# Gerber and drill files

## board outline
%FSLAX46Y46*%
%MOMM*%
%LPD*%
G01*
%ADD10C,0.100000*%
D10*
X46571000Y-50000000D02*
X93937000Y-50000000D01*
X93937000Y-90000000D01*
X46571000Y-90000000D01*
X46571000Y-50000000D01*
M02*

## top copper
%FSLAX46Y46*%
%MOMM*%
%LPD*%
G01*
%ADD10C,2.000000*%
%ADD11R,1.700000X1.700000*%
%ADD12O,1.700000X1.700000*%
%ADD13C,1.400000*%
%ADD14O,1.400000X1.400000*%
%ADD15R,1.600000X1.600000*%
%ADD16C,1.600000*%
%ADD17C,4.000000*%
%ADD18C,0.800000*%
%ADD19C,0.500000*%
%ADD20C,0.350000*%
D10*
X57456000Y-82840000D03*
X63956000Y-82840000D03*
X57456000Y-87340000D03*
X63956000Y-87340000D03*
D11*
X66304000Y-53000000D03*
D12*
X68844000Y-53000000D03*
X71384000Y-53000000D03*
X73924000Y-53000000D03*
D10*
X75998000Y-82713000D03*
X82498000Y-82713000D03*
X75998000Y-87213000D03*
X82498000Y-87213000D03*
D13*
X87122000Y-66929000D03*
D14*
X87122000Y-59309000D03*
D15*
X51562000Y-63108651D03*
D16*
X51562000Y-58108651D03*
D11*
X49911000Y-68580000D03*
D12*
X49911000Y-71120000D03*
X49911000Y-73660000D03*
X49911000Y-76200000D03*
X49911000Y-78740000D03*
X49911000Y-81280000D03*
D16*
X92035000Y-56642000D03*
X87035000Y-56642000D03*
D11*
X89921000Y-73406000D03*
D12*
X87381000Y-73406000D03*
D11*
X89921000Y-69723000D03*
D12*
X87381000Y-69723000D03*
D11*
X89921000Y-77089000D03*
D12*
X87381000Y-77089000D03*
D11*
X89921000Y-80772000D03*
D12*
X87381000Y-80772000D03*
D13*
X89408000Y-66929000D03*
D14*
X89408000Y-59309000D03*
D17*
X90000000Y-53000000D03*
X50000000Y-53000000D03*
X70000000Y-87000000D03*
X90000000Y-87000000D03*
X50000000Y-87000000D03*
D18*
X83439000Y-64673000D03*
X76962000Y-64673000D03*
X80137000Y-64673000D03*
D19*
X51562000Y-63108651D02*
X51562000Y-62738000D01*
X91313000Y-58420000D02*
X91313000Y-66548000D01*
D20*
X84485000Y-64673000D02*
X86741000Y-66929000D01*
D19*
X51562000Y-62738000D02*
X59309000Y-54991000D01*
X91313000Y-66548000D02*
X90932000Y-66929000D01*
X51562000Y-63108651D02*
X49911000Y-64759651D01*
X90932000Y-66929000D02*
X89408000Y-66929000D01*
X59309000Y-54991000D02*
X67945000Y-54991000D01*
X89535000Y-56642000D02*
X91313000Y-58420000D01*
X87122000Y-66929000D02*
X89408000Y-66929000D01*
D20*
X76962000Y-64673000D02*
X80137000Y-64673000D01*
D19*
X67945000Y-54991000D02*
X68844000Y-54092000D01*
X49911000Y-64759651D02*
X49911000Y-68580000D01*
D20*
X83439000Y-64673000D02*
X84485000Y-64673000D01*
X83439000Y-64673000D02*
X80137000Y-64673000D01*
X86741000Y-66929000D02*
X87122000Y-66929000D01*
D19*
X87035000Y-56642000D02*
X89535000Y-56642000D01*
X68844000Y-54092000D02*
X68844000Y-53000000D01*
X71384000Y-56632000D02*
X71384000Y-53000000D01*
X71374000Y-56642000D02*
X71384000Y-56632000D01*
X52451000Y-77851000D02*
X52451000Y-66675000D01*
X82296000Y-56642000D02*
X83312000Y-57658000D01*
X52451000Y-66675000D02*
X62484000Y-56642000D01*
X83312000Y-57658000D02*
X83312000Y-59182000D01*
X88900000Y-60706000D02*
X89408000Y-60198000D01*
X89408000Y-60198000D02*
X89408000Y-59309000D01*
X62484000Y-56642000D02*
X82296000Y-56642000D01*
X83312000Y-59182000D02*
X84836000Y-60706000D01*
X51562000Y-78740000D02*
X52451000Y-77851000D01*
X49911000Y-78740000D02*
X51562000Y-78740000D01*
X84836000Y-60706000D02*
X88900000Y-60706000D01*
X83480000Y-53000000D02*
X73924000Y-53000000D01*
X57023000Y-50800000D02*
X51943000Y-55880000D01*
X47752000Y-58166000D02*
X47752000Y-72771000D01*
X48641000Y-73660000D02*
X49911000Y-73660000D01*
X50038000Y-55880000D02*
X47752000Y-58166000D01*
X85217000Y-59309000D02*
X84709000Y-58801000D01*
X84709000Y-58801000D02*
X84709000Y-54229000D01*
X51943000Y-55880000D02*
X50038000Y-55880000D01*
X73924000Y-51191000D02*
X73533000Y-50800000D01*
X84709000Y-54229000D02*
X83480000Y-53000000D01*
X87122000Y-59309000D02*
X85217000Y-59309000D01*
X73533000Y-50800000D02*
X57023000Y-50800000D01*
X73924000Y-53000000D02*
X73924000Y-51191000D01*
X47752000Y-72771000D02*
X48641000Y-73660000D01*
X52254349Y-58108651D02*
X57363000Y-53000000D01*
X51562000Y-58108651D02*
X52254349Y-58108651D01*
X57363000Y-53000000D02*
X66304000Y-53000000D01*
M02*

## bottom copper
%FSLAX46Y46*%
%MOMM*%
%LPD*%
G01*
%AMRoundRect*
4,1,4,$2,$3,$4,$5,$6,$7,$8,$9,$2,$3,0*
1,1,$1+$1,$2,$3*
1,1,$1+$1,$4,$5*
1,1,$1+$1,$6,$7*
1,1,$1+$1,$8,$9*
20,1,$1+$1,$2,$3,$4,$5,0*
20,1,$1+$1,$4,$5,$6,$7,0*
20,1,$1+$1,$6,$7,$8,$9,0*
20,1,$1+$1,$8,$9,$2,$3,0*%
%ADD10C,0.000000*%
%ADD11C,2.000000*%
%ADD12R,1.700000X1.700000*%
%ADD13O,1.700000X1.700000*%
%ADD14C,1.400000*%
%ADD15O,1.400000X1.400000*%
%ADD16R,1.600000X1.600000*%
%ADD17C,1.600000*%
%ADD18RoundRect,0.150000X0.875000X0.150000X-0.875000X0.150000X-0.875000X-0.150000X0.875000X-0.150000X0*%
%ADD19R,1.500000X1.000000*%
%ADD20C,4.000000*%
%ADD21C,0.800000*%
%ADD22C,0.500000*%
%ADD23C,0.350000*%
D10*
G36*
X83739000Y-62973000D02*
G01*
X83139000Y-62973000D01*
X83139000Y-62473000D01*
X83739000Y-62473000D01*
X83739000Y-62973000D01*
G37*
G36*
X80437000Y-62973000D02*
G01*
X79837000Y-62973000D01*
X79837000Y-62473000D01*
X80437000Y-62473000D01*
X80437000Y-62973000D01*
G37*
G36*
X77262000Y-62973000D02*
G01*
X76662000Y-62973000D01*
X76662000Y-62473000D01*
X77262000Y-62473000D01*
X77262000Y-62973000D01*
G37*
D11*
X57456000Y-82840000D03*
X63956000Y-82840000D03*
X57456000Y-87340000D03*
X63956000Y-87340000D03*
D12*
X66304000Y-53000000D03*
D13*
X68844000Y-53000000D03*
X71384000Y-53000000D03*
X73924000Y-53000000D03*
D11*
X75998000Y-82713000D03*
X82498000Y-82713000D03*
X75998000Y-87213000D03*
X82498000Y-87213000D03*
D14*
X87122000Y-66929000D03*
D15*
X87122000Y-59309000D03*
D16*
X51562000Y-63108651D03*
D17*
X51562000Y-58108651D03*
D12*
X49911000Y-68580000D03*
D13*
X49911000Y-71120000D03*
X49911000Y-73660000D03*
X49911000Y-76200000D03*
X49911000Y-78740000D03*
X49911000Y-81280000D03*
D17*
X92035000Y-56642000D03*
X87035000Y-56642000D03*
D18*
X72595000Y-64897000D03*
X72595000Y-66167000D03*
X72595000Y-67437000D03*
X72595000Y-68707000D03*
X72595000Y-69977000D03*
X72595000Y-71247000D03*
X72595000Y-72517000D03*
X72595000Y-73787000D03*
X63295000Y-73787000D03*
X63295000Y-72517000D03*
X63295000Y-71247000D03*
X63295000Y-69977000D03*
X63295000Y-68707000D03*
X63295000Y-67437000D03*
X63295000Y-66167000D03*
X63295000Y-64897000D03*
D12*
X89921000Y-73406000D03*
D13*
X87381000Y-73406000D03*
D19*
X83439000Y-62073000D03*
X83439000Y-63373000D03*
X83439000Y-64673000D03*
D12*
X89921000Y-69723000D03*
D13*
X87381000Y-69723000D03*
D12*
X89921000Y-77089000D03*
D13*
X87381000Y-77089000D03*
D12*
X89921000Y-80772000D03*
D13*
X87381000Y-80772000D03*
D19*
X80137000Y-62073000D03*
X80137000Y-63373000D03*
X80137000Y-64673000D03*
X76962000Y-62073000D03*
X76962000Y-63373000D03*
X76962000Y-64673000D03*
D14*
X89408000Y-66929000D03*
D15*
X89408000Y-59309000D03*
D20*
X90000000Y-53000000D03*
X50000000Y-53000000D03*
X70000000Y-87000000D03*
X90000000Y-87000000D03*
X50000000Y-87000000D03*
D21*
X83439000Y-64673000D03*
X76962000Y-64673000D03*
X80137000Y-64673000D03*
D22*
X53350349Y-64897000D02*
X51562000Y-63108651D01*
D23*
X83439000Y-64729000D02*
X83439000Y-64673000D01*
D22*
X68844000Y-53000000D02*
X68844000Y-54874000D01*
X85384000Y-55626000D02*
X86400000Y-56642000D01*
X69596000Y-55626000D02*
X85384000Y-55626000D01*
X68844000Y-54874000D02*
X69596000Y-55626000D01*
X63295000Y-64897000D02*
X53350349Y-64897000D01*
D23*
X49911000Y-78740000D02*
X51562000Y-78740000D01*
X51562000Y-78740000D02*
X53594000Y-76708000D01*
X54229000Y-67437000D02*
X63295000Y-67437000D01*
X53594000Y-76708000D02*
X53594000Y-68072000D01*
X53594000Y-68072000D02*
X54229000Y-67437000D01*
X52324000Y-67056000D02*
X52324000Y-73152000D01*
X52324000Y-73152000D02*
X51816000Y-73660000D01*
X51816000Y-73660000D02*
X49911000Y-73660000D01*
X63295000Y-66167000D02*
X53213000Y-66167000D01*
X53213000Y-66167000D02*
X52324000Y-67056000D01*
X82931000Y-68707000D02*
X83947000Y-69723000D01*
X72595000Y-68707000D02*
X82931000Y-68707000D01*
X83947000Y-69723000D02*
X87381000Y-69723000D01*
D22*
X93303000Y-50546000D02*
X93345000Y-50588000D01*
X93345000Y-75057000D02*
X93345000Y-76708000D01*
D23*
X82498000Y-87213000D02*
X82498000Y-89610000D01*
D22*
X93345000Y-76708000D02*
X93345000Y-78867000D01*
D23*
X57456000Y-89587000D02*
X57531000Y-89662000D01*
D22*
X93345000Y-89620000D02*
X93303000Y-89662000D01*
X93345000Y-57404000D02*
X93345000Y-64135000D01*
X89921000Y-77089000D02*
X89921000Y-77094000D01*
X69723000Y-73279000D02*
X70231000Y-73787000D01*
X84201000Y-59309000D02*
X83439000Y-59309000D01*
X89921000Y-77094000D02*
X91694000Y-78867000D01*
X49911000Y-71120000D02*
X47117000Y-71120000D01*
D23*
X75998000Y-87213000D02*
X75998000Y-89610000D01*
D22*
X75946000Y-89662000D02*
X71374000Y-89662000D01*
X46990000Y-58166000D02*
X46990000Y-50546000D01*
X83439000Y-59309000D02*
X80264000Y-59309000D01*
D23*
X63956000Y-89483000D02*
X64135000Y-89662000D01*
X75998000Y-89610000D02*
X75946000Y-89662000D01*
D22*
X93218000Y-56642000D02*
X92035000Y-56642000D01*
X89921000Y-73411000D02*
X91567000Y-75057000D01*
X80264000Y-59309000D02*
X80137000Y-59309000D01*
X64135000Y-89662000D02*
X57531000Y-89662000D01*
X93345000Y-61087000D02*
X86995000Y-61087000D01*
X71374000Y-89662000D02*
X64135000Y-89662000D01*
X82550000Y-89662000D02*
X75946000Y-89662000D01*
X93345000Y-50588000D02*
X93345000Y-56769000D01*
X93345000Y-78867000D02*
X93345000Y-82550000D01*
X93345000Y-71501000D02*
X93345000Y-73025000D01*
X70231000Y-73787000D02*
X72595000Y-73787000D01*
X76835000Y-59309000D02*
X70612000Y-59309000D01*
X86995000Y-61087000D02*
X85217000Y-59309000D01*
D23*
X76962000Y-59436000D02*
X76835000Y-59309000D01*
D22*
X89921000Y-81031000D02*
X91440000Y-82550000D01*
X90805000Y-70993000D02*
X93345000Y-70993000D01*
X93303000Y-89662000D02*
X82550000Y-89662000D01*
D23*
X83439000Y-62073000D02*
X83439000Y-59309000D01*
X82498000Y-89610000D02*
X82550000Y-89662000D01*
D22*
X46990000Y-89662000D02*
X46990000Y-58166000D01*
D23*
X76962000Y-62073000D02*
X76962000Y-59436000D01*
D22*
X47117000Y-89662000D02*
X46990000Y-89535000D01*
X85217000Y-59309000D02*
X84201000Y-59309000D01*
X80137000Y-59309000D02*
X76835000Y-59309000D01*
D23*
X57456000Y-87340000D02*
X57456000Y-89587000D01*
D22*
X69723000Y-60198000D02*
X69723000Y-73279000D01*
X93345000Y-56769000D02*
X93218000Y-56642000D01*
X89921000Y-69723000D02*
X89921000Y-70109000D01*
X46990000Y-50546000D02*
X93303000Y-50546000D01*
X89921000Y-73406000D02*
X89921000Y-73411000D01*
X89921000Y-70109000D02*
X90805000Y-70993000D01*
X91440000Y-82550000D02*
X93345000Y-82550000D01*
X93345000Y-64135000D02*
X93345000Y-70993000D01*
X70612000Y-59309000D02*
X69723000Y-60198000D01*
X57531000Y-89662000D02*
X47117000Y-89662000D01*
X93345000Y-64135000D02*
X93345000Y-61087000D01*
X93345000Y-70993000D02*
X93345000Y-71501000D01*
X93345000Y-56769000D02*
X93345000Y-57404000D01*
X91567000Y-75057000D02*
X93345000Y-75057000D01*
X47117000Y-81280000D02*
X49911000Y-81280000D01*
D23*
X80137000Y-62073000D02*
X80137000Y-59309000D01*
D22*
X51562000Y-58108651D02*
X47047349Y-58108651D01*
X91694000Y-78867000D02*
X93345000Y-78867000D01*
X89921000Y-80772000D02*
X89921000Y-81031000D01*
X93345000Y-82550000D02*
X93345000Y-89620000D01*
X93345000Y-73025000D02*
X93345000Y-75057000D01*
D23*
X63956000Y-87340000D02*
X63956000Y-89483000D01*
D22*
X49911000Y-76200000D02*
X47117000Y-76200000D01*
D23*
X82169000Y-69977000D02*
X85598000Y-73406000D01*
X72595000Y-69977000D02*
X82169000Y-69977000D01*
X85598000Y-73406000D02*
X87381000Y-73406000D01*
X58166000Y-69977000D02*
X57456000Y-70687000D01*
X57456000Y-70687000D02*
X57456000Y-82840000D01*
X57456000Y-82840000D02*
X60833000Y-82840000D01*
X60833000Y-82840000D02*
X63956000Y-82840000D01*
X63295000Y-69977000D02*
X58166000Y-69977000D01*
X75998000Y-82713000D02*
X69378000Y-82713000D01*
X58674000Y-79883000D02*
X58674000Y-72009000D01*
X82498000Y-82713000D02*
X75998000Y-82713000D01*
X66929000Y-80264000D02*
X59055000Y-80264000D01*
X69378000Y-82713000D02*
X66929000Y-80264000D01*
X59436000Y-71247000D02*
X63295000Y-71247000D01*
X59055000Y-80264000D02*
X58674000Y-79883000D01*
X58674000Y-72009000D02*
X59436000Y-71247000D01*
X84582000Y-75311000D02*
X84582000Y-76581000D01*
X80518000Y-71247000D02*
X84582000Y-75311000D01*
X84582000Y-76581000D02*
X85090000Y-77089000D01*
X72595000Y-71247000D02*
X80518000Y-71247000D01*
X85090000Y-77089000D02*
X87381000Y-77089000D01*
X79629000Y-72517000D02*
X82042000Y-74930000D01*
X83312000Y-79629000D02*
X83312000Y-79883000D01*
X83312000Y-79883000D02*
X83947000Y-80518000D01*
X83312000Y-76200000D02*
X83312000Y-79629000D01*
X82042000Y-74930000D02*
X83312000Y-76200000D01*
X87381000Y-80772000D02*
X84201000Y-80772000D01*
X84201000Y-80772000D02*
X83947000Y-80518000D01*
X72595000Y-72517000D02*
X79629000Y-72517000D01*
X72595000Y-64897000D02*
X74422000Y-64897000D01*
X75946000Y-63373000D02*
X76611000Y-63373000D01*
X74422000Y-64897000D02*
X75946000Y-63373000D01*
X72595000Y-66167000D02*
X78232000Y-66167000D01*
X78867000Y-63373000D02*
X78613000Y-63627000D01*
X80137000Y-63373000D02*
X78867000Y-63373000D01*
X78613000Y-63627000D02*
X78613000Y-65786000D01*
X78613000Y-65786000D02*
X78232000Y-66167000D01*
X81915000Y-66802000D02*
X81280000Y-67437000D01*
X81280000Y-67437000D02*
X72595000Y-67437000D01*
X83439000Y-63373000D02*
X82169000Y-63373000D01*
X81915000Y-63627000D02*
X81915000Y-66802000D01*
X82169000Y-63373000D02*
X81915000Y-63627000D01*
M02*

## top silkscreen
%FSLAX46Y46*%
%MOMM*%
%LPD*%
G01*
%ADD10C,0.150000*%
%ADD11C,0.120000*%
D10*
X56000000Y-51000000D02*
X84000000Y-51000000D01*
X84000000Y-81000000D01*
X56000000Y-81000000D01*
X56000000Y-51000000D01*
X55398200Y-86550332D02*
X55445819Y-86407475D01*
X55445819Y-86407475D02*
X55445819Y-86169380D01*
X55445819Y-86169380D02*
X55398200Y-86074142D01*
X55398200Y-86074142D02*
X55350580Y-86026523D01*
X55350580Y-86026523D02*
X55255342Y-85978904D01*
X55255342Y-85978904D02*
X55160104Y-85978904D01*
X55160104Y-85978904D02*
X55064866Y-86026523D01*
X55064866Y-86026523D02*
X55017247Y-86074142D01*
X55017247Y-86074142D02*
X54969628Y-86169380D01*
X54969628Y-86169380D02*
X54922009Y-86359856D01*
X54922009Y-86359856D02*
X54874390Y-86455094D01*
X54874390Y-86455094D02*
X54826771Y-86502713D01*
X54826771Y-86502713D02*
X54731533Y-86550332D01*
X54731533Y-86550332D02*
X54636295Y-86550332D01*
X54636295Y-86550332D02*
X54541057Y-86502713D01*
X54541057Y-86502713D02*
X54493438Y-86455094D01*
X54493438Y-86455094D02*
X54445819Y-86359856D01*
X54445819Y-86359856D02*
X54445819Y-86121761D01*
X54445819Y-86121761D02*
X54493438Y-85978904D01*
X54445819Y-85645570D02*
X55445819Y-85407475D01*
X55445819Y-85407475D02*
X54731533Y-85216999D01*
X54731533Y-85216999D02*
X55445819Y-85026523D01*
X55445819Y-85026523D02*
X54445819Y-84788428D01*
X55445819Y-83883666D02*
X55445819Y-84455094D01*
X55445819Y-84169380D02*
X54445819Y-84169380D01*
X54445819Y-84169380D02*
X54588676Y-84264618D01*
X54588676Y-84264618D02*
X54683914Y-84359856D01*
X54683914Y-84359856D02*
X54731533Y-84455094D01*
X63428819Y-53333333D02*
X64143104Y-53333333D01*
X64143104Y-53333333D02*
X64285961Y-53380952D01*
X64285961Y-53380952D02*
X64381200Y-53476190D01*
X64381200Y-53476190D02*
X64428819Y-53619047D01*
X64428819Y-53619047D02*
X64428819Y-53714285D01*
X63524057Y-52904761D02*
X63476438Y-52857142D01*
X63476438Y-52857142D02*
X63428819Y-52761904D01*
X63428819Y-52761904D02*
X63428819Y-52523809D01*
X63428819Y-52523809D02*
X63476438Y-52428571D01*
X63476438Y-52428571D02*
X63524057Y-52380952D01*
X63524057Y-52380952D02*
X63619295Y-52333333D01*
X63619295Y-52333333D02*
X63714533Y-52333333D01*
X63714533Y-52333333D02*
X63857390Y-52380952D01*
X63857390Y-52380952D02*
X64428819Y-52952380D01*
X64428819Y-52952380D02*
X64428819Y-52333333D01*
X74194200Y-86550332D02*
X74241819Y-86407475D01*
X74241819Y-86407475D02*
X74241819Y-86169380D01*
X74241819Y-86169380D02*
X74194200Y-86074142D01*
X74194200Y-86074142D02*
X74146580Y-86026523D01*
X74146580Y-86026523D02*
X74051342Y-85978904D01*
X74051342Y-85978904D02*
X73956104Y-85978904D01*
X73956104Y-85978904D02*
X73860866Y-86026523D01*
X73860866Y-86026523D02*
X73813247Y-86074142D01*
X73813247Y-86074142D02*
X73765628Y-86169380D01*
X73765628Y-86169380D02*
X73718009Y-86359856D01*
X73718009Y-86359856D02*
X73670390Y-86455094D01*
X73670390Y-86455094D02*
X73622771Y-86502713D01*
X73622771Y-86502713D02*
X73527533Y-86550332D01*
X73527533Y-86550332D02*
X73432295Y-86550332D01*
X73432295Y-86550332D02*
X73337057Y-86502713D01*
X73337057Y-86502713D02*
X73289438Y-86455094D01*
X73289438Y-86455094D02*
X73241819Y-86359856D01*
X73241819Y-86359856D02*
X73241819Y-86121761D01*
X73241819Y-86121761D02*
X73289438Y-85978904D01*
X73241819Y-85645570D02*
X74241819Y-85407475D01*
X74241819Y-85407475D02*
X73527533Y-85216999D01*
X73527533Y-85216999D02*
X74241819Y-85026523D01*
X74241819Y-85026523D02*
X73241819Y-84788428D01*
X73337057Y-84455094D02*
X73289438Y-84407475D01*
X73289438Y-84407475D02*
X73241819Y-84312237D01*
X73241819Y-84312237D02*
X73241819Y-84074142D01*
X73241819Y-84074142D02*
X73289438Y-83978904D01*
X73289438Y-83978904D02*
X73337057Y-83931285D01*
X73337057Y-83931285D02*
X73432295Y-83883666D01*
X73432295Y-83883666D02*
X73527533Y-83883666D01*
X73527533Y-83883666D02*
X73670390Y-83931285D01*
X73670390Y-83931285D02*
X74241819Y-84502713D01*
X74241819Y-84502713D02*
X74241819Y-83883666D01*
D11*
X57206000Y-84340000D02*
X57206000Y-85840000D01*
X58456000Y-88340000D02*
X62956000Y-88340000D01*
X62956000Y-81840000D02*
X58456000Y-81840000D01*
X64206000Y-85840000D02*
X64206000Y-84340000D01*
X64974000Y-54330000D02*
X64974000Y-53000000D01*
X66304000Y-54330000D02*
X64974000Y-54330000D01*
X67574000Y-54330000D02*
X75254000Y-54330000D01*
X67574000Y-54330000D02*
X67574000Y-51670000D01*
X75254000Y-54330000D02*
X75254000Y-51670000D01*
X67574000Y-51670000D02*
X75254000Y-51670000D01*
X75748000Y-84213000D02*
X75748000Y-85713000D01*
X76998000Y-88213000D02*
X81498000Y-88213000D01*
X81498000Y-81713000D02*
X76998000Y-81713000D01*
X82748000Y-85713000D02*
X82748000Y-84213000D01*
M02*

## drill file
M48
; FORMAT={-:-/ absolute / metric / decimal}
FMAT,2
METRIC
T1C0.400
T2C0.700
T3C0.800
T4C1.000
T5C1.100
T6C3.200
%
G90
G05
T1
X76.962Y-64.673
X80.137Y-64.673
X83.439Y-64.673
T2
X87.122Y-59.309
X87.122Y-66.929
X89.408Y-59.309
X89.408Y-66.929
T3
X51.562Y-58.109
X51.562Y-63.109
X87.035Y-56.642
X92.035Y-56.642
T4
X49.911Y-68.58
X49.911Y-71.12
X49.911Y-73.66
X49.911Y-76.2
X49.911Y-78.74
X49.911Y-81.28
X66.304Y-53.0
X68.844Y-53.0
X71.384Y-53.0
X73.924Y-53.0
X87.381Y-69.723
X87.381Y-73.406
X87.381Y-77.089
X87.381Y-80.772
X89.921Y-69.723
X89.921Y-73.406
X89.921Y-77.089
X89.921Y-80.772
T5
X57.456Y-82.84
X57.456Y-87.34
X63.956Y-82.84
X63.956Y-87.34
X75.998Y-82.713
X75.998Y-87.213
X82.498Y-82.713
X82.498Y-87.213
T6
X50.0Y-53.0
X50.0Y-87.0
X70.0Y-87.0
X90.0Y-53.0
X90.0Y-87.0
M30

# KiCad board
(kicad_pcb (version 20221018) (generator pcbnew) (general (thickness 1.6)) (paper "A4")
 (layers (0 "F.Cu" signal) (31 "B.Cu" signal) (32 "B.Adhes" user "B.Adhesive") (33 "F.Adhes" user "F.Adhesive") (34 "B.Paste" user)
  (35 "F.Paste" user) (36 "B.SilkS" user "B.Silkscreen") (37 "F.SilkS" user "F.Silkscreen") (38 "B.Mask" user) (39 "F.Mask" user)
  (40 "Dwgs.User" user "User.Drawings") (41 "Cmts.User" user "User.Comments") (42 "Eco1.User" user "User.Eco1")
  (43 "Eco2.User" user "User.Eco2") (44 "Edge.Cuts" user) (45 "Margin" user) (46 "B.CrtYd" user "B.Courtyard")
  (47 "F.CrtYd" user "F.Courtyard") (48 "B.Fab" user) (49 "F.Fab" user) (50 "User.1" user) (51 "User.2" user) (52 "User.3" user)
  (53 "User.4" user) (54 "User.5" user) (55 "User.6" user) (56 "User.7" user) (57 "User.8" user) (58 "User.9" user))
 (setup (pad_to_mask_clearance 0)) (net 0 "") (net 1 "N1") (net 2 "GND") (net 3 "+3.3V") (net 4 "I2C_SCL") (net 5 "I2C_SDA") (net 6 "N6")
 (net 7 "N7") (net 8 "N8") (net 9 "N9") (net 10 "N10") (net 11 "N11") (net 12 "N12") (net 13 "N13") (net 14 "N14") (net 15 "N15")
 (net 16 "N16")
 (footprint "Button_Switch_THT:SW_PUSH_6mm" (layer "F.Cu") (at 57.456 82.84)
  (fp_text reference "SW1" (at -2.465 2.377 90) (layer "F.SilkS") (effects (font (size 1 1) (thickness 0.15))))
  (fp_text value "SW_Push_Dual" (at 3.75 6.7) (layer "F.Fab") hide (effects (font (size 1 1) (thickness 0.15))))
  (fp_line (start -0.25 1.5) (end -0.25 3) (stroke (width 0.12) (type solid)) (layer "F.SilkS"))
  (fp_line (start 1 5.5) (end 5.5 5.5) (stroke (width 0.12) (type solid)) (layer "F.SilkS"))
  (fp_line (start 5.5 -1) (end 1 -1) (stroke (width 0.12) (type solid)) (layer "F.SilkS"))
  (fp_line (start 6.75 3) (end 6.75 1.5) (stroke (width 0.12) (type solid)) (layer "F.SilkS"))
  (pad "1" thru_hole circle (at 0 0 90) (size 2 2) (drill 1.1) (layers "*.Cu" "*.Mask") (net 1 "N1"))
  (pad "1" thru_hole circle (at 6.5 0 90) (size 2 2) (drill 1.1) (layers "*.Cu" "*.Mask") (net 1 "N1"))
  (pad "2" thru_hole circle (at 0 4.5 90) (size 2 2) (drill 1.1) (layers "*.Cu" "*.Mask") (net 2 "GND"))
  (pad "2" thru_hole circle (at 6.5 4.5 90) (size 2 2) (drill 1.1) (layers "*.Cu" "*.Mask") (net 2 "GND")))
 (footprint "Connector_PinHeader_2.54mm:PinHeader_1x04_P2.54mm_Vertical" (layer "F.Cu") (at 66.304 53 90)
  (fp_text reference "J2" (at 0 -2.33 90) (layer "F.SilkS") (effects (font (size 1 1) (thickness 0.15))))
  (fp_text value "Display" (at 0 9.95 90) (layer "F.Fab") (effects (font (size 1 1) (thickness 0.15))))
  (fp_line (start -1.33 -1.33) (end 0 -1.33) (stroke (width 0.12) (type solid)) (layer "F.SilkS"))
  (fp_line (start -1.33 0) (end -1.33 -1.33) (stroke (width 0.12) (type solid)) (layer "F.SilkS"))
  (fp_line (start -1.33 1.27) (end -1.33 8.95) (stroke (width 0.12) (type solid)) (layer "F.SilkS"))
  (fp_line (start -1.33 1.27) (end 1.33 1.27) (stroke (width 0.12) (type solid)) (layer "F.SilkS"))
  (fp_line (start -1.33 8.95) (end 1.33 8.95) (stroke (width 0.12) (type solid)) (layer "F.SilkS"))
  (fp_line (start 1.33 1.27) (end 1.33 8.95) (stroke (width 0.12) (type solid)) (layer "F.SilkS"))
  (pad "1" thru_hole rect (at 0 0 90) (size 1.7 1.7) (drill 1) (layers "*.Cu" "*.Mask") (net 2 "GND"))
  (pad "2" thru_hole oval (at 0 2.54 90) (size 1.7 1.7) (drill 1) (layers "*.Cu" "*.Mask") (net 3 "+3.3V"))
  (pad "3" thru_hole oval (at 0 5.08 90) (size 1.7 1.7) (drill 1) (layers "*.Cu" "*.Mask") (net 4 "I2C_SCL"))
  (pad "4" thru_hole oval (at 0 7.62 90) (size 1.7 1.7) (drill 1) (layers "*.Cu" "*.Mask") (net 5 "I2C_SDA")))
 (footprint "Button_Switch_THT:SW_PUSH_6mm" (layer "F.Cu") (at 75.998 82.713)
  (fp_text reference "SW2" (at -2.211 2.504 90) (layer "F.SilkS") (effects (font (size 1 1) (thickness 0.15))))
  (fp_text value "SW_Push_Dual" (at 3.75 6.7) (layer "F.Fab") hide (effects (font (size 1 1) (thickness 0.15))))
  (fp_line (start -0.25 1.5) (end -0.25 3) (stroke (width 0.12) (type solid)) (layer "F.SilkS"))
  (fp_line (start 1 5.5) (end 5.5 5.5) (stroke (width 0.12) (type solid)) (layer "F.SilkS"))
  (fp_line (start 5.5 -1) (end 1 -1) (stroke (width 0.12) (type solid)) (layer "F.SilkS"))
  (fp_line (start 6.75 3) (end 6.75 1.5) (stroke (width 0.12) (type solid)) (layer "F.SilkS"))
  (pad "1" thru_hole circle (at 0 0 90) (size 2 2) (drill 1.1) (layers "*.Cu" "*.Mask") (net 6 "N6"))
  (pad "1" thru_hole circle (at 6.5 0 90) (size 2 2) (drill 1.1) (layers "*.Cu" "*.Mask") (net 6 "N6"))
  (pad "2" thru_hole circle (at 0 4.5 90) (size 2 2) (drill 1.1) (layers "*.Cu" "*.Mask") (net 2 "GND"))
  (pad "2" thru_hole circle (at 6.5 4.5 90) (size 2 2) (drill 1.1) (layers "*.Cu" "*.Mask") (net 2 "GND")))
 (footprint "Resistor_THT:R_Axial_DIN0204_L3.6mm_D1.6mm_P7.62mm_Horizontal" (layer "B.Cu") (at 87.122 66.929 90)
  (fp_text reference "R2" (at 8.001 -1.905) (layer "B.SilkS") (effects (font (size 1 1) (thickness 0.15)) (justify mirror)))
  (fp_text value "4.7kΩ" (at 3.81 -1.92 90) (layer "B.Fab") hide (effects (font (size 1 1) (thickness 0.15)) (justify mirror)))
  (pad "1" thru_hole circle (at 0 0 90) (size 1.4 1.4) (drill 0.7) (layers "*.Cu" "*.Mask") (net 3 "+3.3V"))
  (pad "2" thru_hole oval (at 7.62 0 90) (size 1.4 1.4) (drill 0.7) (layers "*.Cu" "*.Mask") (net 5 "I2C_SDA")))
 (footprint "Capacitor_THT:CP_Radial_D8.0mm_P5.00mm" (layer "B.Cu") (at 51.562 63.108651 90)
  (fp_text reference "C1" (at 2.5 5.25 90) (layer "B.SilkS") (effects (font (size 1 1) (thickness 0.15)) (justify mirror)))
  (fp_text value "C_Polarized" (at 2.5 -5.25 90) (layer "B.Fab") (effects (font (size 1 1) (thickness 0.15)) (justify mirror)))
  (pad "1" thru_hole rect (at 0 0 90) (size 1.6 1.6) (drill 0.8) (layers "*.Cu" "*.Mask") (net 3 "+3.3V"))
  (pad "2" thru_hole circle (at 5 0 90) (size 1.6 1.6) (drill 0.8) (layers "*.Cu" "*.Mask") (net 2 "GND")))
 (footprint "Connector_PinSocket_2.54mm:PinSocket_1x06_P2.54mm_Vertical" (layer "B.Cu") (at 49.911 68.58 180)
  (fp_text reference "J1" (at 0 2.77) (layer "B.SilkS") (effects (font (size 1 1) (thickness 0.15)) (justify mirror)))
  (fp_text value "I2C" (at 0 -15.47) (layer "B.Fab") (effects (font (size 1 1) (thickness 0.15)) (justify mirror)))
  (pad "1" thru_hole rect (at 0 0 180) (size 1.7 1.7) (drill 1) (layers "*.Cu" "*.Mask") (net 3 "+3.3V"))
  (pad "2" thru_hole oval (at 0 -2.54 180) (size 1.7 1.7) (drill 1) (layers "*.Cu" "*.Mask") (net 2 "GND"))
  (pad "3" thru_hole oval (at 0 -5.08 180) (size 1.7 1.7) (drill 1) (layers "*.Cu" "*.Mask") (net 5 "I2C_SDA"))
  (pad "4" thru_hole oval (at 0 -7.62 180) (size 1.7 1.7) (drill 1) (layers "*.Cu" "*.Mask") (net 2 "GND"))
  (pad "5" thru_hole oval (at 0 -10.16 180) (size 1.7 1.7) (drill 1) (layers "*.Cu" "*.Mask") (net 4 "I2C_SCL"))
  (pad "6" thru_hole oval (at 0 -12.7 180) (size 1.7 1.7) (drill 1) (layers "*.Cu" "*.Mask") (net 2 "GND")))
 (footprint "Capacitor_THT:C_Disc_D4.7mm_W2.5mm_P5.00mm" (layer "B.Cu") (at 92.035 56.642 180)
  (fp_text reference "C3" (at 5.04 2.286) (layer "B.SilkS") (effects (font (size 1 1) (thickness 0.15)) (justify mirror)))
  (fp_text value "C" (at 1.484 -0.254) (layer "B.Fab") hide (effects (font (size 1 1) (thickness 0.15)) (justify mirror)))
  (pad "1" thru_hole circle (at 0 0 180) (size 1.6 1.6) (drill 0.8) (layers "*.Cu" "*.Mask") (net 2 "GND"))
  (pad "2" thru_hole circle (at 5 0 180) (size 1.6 1.6) (drill 0.8) (layers "*.Cu" "*.Mask") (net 3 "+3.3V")))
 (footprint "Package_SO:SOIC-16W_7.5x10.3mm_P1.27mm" (layer "B.Cu") (at 67.945 69.342 180)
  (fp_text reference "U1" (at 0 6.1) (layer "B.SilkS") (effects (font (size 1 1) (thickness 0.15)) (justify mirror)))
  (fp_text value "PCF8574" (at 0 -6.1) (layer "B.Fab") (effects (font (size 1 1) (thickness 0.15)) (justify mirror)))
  (pad "1" smd roundrect (at -4.65 4.445 180) (size 2.05 0.6) (layers "B.Cu" "B.Paste" "B.Mask") (roundrect_rratio 0.25) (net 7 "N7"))
  (pad "2" smd roundrect (at -4.65 3.175 180) (size 2.05 0.6) (layers "B.Cu" "B.Paste" "B.Mask") (roundrect_rratio 0.25) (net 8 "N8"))
  (pad "3" smd roundrect (at -4.65 1.905 180) (size 2.05 0.6) (layers "B.Cu" "B.Paste" "B.Mask") (roundrect_rratio 0.25) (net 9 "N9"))
  (pad "4" smd roundrect (at -4.65 0.635 180) (size 2.05 0.6) (layers "B.Cu" "B.Paste" "B.Mask") (roundrect_rratio 0.25) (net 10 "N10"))
  (pad "5" smd roundrect (at -4.65 -0.635 180) (size 2.05 0.6) (layers "B.Cu" "B.Paste" "B.Mask") (roundrect_rratio 0.25) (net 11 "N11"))
  (pad "6" smd roundrect (at -4.65 -1.905 180) (size 2.05 0.6) (layers "B.Cu" "B.Paste" "B.Mask") (roundrect_rratio 0.25) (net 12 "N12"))
  (pad "7" smd roundrect (at -4.65 -3.175 180) (size 2.05 0.6) (layers "B.Cu" "B.Paste" "B.Mask") (roundrect_rratio 0.25) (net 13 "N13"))
  (pad "8" smd roundrect (at -4.65 -4.445 180) (size 2.05 0.6) (layers "B.Cu" "B.Paste" "B.Mask") (roundrect_rratio 0.25) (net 2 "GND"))
  (pad "9" smd roundrect (at 4.65 -4.445 180) (size 2.05 0.6) (layers "B.Cu" "B.Paste" "B.Mask") (roundrect_rratio 0.25) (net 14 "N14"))
  (pad "10" smd roundrect (at 4.65 -3.175 180) (size 2.05 0.6) (layers "B.Cu" "B.Paste" "B.Mask") (roundrect_rratio 0.25) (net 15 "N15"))
  (pad "11" smd roundrect (at 4.65 -1.905 180) (size 2.05 0.6) (layers "B.Cu" "B.Paste" "B.Mask") (roundrect_rratio 0.25) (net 6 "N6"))
  (pad "12" smd roundrect (at 4.65 -0.635 180) (size 2.05 0.6) (layers "B.Cu" "B.Paste" "B.Mask") (roundrect_rratio 0.25) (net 1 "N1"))
  (pad "13" smd roundrect (at 4.65 0.635 180) (size 2.05 0.6) (layers "B.Cu" "B.Paste" "B.Mask") (roundrect_rratio 0.25) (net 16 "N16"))
  (pad "14" smd roundrect (at 4.65 1.905 180) (size 2.05 0.6) (layers "B.Cu" "B.Paste" "B.Mask") (roundrect_rratio 0.25) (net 4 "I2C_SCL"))
  (pad "15" smd roundrect (at 4.65 3.175 180) (size 2.05 0.6) (layers "B.Cu" "B.Paste" "B.Mask") (roundrect_rratio 0.25) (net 5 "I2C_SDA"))
  (pad "16" smd roundrect (at 4.65 4.445 180) (size 2.05 0.6) (layers "B.Cu" "B.Paste" "B.Mask") (roundrect_rratio 0.25) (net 3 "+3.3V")))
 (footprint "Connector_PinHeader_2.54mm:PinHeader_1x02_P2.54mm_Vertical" (layer "B.Cu") (at 89.921 73.406 90)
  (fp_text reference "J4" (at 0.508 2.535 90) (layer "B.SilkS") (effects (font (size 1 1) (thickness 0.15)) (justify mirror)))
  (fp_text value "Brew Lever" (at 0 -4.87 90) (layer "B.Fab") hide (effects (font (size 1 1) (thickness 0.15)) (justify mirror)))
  (pad "1" thru_hole rect (at 0 0 90) (size 1.7 1.7) (drill 1) (layers "*.Cu" "*.Mask") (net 2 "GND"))
  (pad "2" thru_hole oval (at 0 -2.54 90) (size 1.7 1.7) (drill 1) (layers "*.Cu" "*.Mask") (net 11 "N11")))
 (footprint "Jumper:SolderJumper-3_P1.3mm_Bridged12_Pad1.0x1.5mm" (layer "B.Cu") (at 83.439 63.373 -90) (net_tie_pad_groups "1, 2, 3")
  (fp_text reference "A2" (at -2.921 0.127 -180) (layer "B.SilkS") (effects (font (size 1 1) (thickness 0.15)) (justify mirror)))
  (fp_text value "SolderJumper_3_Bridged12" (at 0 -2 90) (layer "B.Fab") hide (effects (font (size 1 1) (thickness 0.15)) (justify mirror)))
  (fp_poly (pts (xy -0.9 0.3) (xy -0.4 0.3) (xy -0.4 -0.3) (xy -0.9 -0.3)) (stroke (width 0) (type solid)) (fill solid) (layer "B.Cu"))
  (pad "1" smd rect (at -1.3 0 270) (size 1 1.5) (layers "B.Cu" "B.Mask") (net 2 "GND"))
  (pad "2" smd rect (at 0 0 270) (size 1 1.5) (layers "B.Cu" "B.Mask") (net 9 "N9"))
  (pad "3" smd rect (at 1.3 0 270) (size 1 1.5) (layers "B.Cu" "B.Mask") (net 3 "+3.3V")))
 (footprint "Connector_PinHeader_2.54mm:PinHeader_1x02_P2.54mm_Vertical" (layer "B.Cu") (at 89.921 69.723 90)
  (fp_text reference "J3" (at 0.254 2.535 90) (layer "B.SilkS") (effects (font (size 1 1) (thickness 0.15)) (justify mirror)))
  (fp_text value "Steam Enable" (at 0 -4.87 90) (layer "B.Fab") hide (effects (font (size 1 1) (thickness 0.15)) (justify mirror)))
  (pad "1" thru_hole rect (at 0 0 90) (size 1.7 1.7) (drill 1) (layers "*.Cu" "*.Mask") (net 2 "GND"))
  (pad "2" thru_hole oval (at 0 -2.54 90) (size 1.7 1.7) (drill 1) (layers "*.Cu" "*.Mask") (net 10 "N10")))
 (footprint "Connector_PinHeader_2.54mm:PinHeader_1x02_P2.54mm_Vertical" (layer "B.Cu") (at 89.921 77.089 90)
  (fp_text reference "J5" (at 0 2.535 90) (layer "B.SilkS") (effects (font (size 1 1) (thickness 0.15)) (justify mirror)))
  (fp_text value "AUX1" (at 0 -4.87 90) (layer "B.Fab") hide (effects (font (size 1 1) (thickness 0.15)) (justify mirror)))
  (pad "1" thru_hole rect (at 0 0 90) (size 1.7 1.7) (drill 1) (layers "*.Cu" "*.Mask") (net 2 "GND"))
  (pad "2" thru_hole oval (at 0 -2.54 90) (size 1.7 1.7) (drill 1) (layers "*.Cu" "*.Mask") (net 12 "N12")))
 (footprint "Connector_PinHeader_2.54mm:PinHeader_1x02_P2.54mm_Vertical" (layer "B.Cu") (at 89.921 80.772 90)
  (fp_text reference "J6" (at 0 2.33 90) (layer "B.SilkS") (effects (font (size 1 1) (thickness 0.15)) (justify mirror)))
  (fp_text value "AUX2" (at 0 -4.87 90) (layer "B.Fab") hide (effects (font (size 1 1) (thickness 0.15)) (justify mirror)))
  (pad "1" thru_hole rect (at 0 0 90) (size 1.7 1.7) (drill 1) (layers "*.Cu" "*.Mask") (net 2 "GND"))
  (pad "2" thru_hole oval (at 0 -2.54 90) (size 1.7 1.7) (drill 1) (layers "*.Cu" "*.Mask") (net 13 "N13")))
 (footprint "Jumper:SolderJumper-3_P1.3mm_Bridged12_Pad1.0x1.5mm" (layer "B.Cu") (at 80.137 63.373 -90) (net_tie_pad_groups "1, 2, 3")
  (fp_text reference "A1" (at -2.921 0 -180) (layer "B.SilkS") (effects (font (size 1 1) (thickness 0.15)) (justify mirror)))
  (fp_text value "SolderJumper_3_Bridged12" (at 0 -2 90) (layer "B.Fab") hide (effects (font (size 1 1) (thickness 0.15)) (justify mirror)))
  (fp_poly (pts (xy -0.9 0.3) (xy -0.4 0.3) (xy -0.4 -0.3) (xy -0.9 -0.3)) (stroke (width 0) (type solid)) (fill solid) (layer "B.Cu"))
  (pad "1" smd rect (at -1.3 0 270) (size 1 1.5) (layers "B.Cu" "B.Mask") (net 2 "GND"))
  (pad "2" smd rect (at 0 0 270) (size 1 1.5) (layers "B.Cu" "B.Mask") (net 8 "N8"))
  (pad "3" smd rect (at 1.3 0 270) (size 1 1.5) (layers "B.Cu" "B.Mask") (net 3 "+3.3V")))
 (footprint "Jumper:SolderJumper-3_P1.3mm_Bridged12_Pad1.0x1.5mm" (layer "B.Cu") (at 76.962 63.373 -90) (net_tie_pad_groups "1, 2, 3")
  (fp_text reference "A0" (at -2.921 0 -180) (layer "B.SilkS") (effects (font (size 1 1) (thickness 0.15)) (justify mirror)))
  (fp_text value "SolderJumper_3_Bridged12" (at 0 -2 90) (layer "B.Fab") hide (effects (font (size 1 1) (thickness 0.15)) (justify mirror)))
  (fp_poly (pts (xy -0.9 0.3) (xy -0.4 0.3) (xy -0.4 -0.3) (xy -0.9 -0.3)) (stroke (width 0) (type solid)) (fill solid) (layer "B.Cu"))
  (pad "1" smd rect (at -1.3 0 270) (size 1 1.5) (layers "B.Cu" "B.Mask") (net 2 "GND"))
  (pad "2" smd rect (at 0 0 270) (size 1 1.5) (layers "B.Cu" "B.Mask") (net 7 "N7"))
  (pad "3" smd rect (at 1.3 0 270) (size 1 1.5) (layers "B.Cu" "B.Mask") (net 3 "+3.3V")))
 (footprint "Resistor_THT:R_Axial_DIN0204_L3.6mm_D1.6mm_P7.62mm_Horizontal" (layer "B.Cu") (at 89.408 66.929 90)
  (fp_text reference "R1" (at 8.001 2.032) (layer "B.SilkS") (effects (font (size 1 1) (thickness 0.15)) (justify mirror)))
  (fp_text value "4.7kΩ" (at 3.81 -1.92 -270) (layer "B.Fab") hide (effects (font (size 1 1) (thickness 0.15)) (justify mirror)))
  (pad "1" thru_hole circle (at 0 0 90) (size 1.4 1.4) (drill 0.7) (layers "*.Cu" "*.Mask") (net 3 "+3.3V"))
  (pad "2" thru_hole oval (at 7.62 0 90) (size 1.4 1.4) (drill 0.7) (layers "*.Cu" "*.Mask") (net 4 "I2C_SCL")))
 (gr_rect (start 56 51) (end 84 81) (stroke (width 0.15) (type default)) (fill none) (layer "F.SilkS"))
 (gr_rect (start 46.571 50) (end 93.937 90) (stroke (width 0.1) (type default)) (fill none) (layer "Edge.Cuts"))
 (via (at 90 53) (size 4) (drill 3.2) (layers "F.Cu" "B.Cu") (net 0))
 (via (at 50 53) (size 4) (drill 3.2) (layers "F.Cu" "B.Cu") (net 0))
 (via (at 70 87) (size 4) (drill 3.2) (layers "F.Cu" "B.Cu") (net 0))
 (via (at 90 87) (size 4) (drill 3.2) (layers "F.Cu" "B.Cu") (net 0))
 (via (at 50 87) (size 4) (drill 3.2) (layers "F.Cu" "B.Cu") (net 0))
 (segment (start 51.562 63.108651) (end 51.562 62.738) (width 0.5) (layer "F.Cu") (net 3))
 (segment (start 91.313 58.42) (end 91.313 66.548) (width 0.5) (layer "F.Cu") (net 3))
 (segment (start 84.485 64.673) (end 86.741 66.929) (width 0.35) (layer "F.Cu") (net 3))
 (segment (start 51.562 62.738) (end 59.309 54.991) (width 0.5) (layer "F.Cu") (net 3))
 (segment (start 91.313 66.548) (end 90.932 66.929) (width 0.5) (layer "F.Cu") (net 3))
 (segment (start 51.562 63.108651) (end 49.911 64.759651) (width 0.5) (layer "F.Cu") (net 3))
 (segment (start 90.932 66.929) (end 89.408 66.929) (width 0.5) (layer "F.Cu") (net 3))
 (segment (start 59.309 54.991) (end 67.945 54.991) (width 0.5) (layer "F.Cu") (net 3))
 (segment (start 89.535 56.642) (end 91.313 58.42) (width 0.5) (layer "F.Cu") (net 3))
 (segment (start 87.122 66.929) (end 89.408 66.929) (width 0.5) (layer "F.Cu") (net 3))
 (segment (start 76.962 64.673) (end 80.137 64.673) (width 0.35) (layer "F.Cu") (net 3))
 (segment (start 67.945 54.991) (end 68.844 54.092) (width 0.5) (layer "F.Cu") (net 3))
 (segment (start 49.911 64.759651) (end 49.911 68.58) (width 0.5) (layer "F.Cu") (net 3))
 (segment (start 83.439 64.673) (end 84.485 64.673) (width 0.35) (layer "F.Cu") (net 3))
 (segment (start 83.439 64.673) (end 80.137 64.673) (width 0.35) (layer "F.Cu") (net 3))
 (segment (start 86.741 66.929) (end 87.122 66.929) (width 0.35) (layer "F.Cu") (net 3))
 (segment (start 87.035 56.642) (end 89.535 56.642) (width 0.5) (layer "F.Cu") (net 3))
 (segment (start 68.844 54.092) (end 68.844 53) (width 0.5) (layer "F.Cu") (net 3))
 (via (at 83.439 64.673) (size 0.8) (drill 0.4) (layers "F.Cu" "B.Cu") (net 3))
 (via (at 76.962 64.673) (size 0.8) (drill 0.4) (layers "F.Cu" "B.Cu") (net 3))
 (via (at 80.137 64.673) (size 0.8) (drill 0.4) (layers "F.Cu" "B.Cu") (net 3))
 (segment (start 53.350349 64.897) (end 51.562 63.108651) (width 0.5) (layer "B.Cu") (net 3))
 (segment (start 83.439 64.729) (end 83.439 64.673) (width 0.35) (layer "B.Cu") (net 3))
 (segment (start 68.844 53) (end 68.844 54.874) (width 0.5) (layer "B.Cu") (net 3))
 (segment (start 85.384 55.626) (end 86.4 56.642) (width 0.5) (layer "B.Cu") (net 3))
 (segment (start 69.596 55.626) (end 85.384 55.626) (width 0.5) (layer "B.Cu") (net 3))
 (segment (start 68.844 54.874) (end 69.596 55.626) (width 0.5) (layer "B.Cu") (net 3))
 (segment (start 63.295 64.897) (end 53.350349 64.897) (width 0.5) (layer "B.Cu") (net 3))
 (segment (start 71.384 56.632) (end 71.384 53) (width 0.5) (layer "F.Cu") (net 4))
 (segment (start 71.374 56.642) (end 71.384 56.632) (width 0.5) (layer "F.Cu") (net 4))
 (segment (start 52.451 77.851) (end 52.451 66.675) (width 0.5) (layer "F.Cu") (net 4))
 (segment (start 82.296 56.642) (end 83.312 57.658) (width 0.5) (layer "F.Cu") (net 4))
 (segment (start 52.451 66.675) (end 62.484 56.642) (width 0.5) (layer "F.Cu") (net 4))
 (segment (start 83.312 57.658) (end 83.312 59.182) (width 0.5) (layer "F.Cu") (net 4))
 (segment (start 88.9 60.706) (end 89.408 60.198) (width 0.5) (layer "F.Cu") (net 4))
 (segment (start 89.408 60.198) (end 89.408 59.309) (width 0.5) (layer "F.Cu") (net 4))
 (segment (start 62.484 56.642) (end 82.296 56.642) (width 0.5) (layer "F.Cu") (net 4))
 (segment (start 83.312 59.182) (end 84.836 60.706) (width 0.5) (layer "F.Cu") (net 4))
 (segment (start 51.562 78.74) (end 52.451 77.851) (width 0.5) (layer "F.Cu") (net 4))
 (segment (start 49.911 78.74) (end 51.562 78.74) (width 0.5) (layer "F.Cu") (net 4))
 (segment (start 84.836 60.706) (end 88.9 60.706) (width 0.5) (layer "F.Cu") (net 4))
 (segment (start 49.911 78.74) (end 51.562 78.74) (width 0.35) (layer "B.Cu") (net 4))
 (segment (start 51.562 78.74) (end 53.594 76.708) (width 0.35) (layer "B.Cu") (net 4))
 (segment (start 54.229 67.437) (end 63.295 67.437) (width 0.35) (layer "B.Cu") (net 4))
 (segment (start 53.594 76.708) (end 53.594 68.072) (width 0.35) (layer "B.Cu") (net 4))
 (segment (start 53.594 68.072) (end 54.229 67.437) (width 0.35) (layer "B.Cu") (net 4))
 (segment (start 83.48 53) (end 73.924 53) (width 0.5) (layer "F.Cu") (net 5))
 (segment (start 57.023 50.8) (end 51.943 55.88) (width 0.5) (layer "F.Cu") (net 5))
 (segment (start 47.752 58.166) (end 47.752 72.771) (width 0.5) (layer "F.Cu") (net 5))
 (segment (start 48.641 73.66) (end 49.911 73.66) (width 0.5) (layer "F.Cu") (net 5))
 (segment (start 50.038 55.88) (end 47.752 58.166) (width 0.5) (layer "F.Cu") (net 5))
 (segment (start 85.217 59.309) (end 84.709 58.801) (width 0.5) (layer "F.Cu") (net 5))
 (segment (start 84.709 58.801) (end 84.709 54.229) (width 0.5) (layer "F.Cu") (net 5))
 (segment (start 51.943 55.88) (end 50.038 55.88) (width 0.5) (layer "F.Cu") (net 5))
 (segment (start 73.924 51.191) (end 73.533 50.8) (width 0.5) (layer "F.Cu") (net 5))
 (segment (start 84.709 54.229) (end 83.48 53) (width 0.5) (layer "F.Cu") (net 5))
 (segment (start 87.122 59.309) (end 85.217 59.309) (width 0.5) (layer "F.Cu") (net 5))
 (segment (start 73.533 50.8) (end 57.023 50.8) (width 0.5) (layer "F.Cu") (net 5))
 (segment (start 73.924 53) (end 73.924 51.191) (width 0.5) (layer "F.Cu") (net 5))
 (segment (start 47.752 72.771) (end 48.641 73.66) (width 0.5) (layer "F.Cu") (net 5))
 (segment (start 52.324 67.056) (end 52.324 73.152) (width 0.35) (layer "B.Cu") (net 5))
 (segment (start 52.324 73.152) (end 51.816 73.66) (width 0.35) (layer "B.Cu") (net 5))
 (segment (start 51.816 73.66) (end 49.911 73.66) (width 0.35) (layer "B.Cu") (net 5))
 (segment (start 63.295 66.167) (end 53.213 66.167) (width 0.35) (layer "B.Cu") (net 5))
 (segment (start 53.213 66.167) (end 52.324 67.056) (width 0.35) (layer "B.Cu") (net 5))
 (segment (start 82.931 68.707) (end 83.947 69.723) (width 0.35) (layer "B.Cu") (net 10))
 (segment (start 72.595 68.707) (end 82.931 68.707) (width 0.35) (layer "B.Cu") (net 10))
 (segment (start 83.947 69.723) (end 87.381 69.723) (width 0.35) (layer "B.Cu") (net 10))
 (segment (start 52.254349 58.108651) (end 57.363 53) (width 0.5) (layer "F.Cu") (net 2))
 (segment (start 51.562 58.108651) (end 52.254349 58.108651) (width 0.5) (layer "F.Cu") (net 2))
 (segment (start 57.363 53) (end 66.304 53) (width 0.5) (layer "F.Cu") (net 2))
 (segment (start 93.303 50.546) (end 93.345 50.588) (width 0.5) (layer "B.Cu") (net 2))
 (segment (start 93.345 75.057) (end 93.345 76.708) (width 0.5) (layer "B.Cu") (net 2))
 (segment (start 82.498 87.213) (end 82.498 89.61) (width 0.35) (layer "B.Cu") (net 2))
 (segment (start 93.345 76.708) (end 93.345 78.867) (width 0.5) (layer "B.Cu") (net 2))
 (segment (start 57.456 89.587) (end 57.531 89.662) (width 0.35) (layer "B.Cu") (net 2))
 (segment (start 93.345 89.62) (end 93.303 89.662) (width 0.5) (layer "B.Cu") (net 2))
 (segment (start 93.345 57.404) (end 93.345 64.135) (width 0.5) (layer "B.Cu") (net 2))
 (segment (start 89.921 77.089) (end 89.921 77.094) (width 0.5) (layer "B.Cu") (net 2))
 (segment (start 69.723 73.279) (end 70.231 73.787) (width 0.5) (layer "B.Cu") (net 2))
 (segment (start 84.201 59.309) (end 83.439 59.309) (width 0.5) (layer "B.Cu") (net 2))
 (segment (start 89.921 77.094) (end 91.694 78.867) (width 0.5) (layer "B.Cu") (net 2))
 (segment (start 49.911 71.12) (end 47.117 71.12) (width 0.5) (layer "B.Cu") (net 2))
 (segment (start 75.998 87.213) (end 75.998 89.61) (width 0.35) (layer "B.Cu") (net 2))
 (segment (start 75.946 89.662) (end 71.374 89.662) (width 0.5) (layer "B.Cu") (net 2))
 (segment (start 46.99 58.166) (end 46.99 50.546) (width 0.5) (layer "B.Cu") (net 2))
 (segment (start 83.439 59.309) (end 80.264 59.309) (width 0.5) (layer "B.Cu") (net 2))
 (segment (start 63.956 89.483) (end 64.135 89.662) (width 0.35) (layer "B.Cu") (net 2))
 (segment (start 75.998 89.61) (end 75.946 89.662) (width 0.35) (layer "B.Cu") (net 2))
 (segment (start 93.218 56.642) (end 92.035 56.642) (width 0.5) (layer "B.Cu") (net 2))
 (segment (start 89.921 73.411) (end 91.567 75.057) (width 0.5) (layer "B.Cu") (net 2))
 (segment (start 80.264 59.309) (end 80.137 59.309) (width 0.5) (layer "B.Cu") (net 2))
 (segment (start 64.135 89.662) (end 57.531 89.662) (width 0.5) (layer "B.Cu") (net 2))
 (segment (start 93.345 61.087) (end 86.995 61.087) (width 0.5) (layer "B.Cu") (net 2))
 (segment (start 71.374 89.662) (end 64.135 89.662) (width 0.5) (layer "B.Cu") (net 2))
 (segment (start 82.55 89.662) (end 75.946 89.662) (width 0.5) (layer "B.Cu") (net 2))
 (segment (start 93.345 50.588) (end 93.345 56.769) (width 0.5) (layer "B.Cu") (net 2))
 (segment (start 93.345 78.867) (end 93.345 82.55) (width 0.5) (layer "B.Cu") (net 2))
 (segment (start 93.345 71.501) (end 93.345 73.025) (width 0.5) (layer "B.Cu") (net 2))
 (segment (start 70.231 73.787) (end 72.595 73.787) (width 0.5) (layer "B.Cu") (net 2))
 (segment (start 76.835 59.309) (end 70.612 59.309) (width 0.5) (layer "B.Cu") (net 2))
 (segment (start 86.995 61.087) (end 85.217 59.309) (width 0.5) (layer "B.Cu") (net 2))
 (segment (start 76.962 59.436) (end 76.835 59.309) (width 0.35) (layer "B.Cu") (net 2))
 (segment (start 89.921 81.031) (end 91.44 82.55) (width 0.5) (layer "B.Cu") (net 2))
 (segment (start 90.805 70.993) (end 93.345 70.993) (width 0.5) (layer "B.Cu") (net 2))
 (segment (start 93.303 89.662) (end 82.55 89.662) (width 0.5) (layer "B.Cu") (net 2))
 (segment (start 83.439 62.073) (end 83.439 59.309) (width 0.35) (layer "B.Cu") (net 2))
 (segment (start 82.498 89.61) (end 82.55 89.662) (width 0.35) (layer "B.Cu") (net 2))
 (segment (start 46.99 89.662) (end 46.99 58.166) (width 0.5) (layer "B.Cu") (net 2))
 (segment (start 76.962 62.073) (end 76.962 59.436) (width 0.35) (layer "B.Cu") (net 2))
 (segment (start 47.117 89.662) (end 46.99 89.535) (width 0.5) (layer "B.Cu") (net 2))
 (segment (start 85.217 59.309) (end 84.201 59.309) (width 0.5) (layer "B.Cu") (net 2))
 (segment (start 80.137 59.309) (end 76.835 59.309) (width 0.5) (layer "B.Cu") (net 2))
 (segment (start 57.456 87.34) (end 57.456 89.587) (width 0.35) (layer "B.Cu") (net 2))
 (segment (start 69.723 60.198) (end 69.723 73.279) (width 0.5) (layer "B.Cu") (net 2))
 (segment (start 93.345 56.769) (end 93.218 56.642) (width 0.5) (layer "B.Cu") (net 2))
 (segment (start 89.921 69.723) (end 89.921 70.109) (width 0.5) (layer "B.Cu") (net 2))
 (segment (start 46.99 50.546) (end 93.303 50.546) (width 0.5) (layer "B.Cu") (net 2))
 (segment (start 89.921 73.406) (end 89.921 73.411) (width 0.5) (layer "B.Cu") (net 2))
 (segment (start 89.921 70.109) (end 90.805 70.993) (width 0.5) (layer "B.Cu") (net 2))
 (segment (start 91.44 82.55) (end 93.345 82.55) (width 0.5) (layer "B.Cu") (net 2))
 (segment (start 93.345 64.135) (end 93.345 70.993) (width 0.5) (layer "B.Cu") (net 2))
 (segment (start 70.612 59.309) (end 69.723 60.198) (width 0.5) (layer "B.Cu") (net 2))
 (segment (start 57.531 89.662) (end 47.117 89.662) (width 0.5) (layer "B.Cu") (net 2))
 (segment (start 93.345 64.135) (end 93.345 61.087) (width 0.5) (layer "B.Cu") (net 2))
 (segment (start 93.345 70.993) (end 93.345 71.501) (width 0.5) (layer "B.Cu") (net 2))
 (segment (start 93.345 56.769) (end 93.345 57.404) (width 0.5) (layer "B.Cu") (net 2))
 (segment (start 91.567 75.057) (end 93.345 75.057) (width 0.5) (layer "B.Cu") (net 2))
 (segment (start 47.117 81.28) (end 49.911 81.28) (width 0.5) (layer "B.Cu") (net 2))
 (segment (start 80.137 62.073) (end 80.137 59.309) (width 0.35) (layer "B.Cu") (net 2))
 (segment (start 51.562 58.108651) (end 47.047349 58.108651) (width 0.5) (layer "B.Cu") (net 2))
 (segment (start 91.694 78.867) (end 93.345 78.867) (width 0.5) (layer "B.Cu") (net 2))
 (segment (start 89.921 80.772) (end 89.921 81.031) (width 0.5) (layer "B.Cu") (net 2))
 (segment (start 93.345 82.55) (end 93.345 89.62) (width 0.5) (layer "B.Cu") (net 2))
 (segment (start 93.345 73.025) (end 93.345 75.057) (width 0.5) (layer "B.Cu") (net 2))
 (segment (start 63.956 87.34) (end 63.956 89.483) (width 0.35) (layer "B.Cu") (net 2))
 (segment (start 49.911 76.2) (end 47.117 76.2) (width 0.5) (layer "B.Cu") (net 2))
 (segment (start 82.169 69.977) (end 85.598 73.406) (width 0.35) (layer "B.Cu") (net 11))
 (segment (start 72.595 69.977) (end 82.169 69.977) (width 0.35) (layer "B.Cu") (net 11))
 (segment (start 85.598 73.406) (end 87.381 73.406) (width 0.35) (layer "B.Cu") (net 11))
 (segment (start 58.166 69.977) (end 57.456 70.687) (width 0.35) (layer "B.Cu") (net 1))
 (segment (start 57.456 70.687) (end 57.456 82.84) (width 0.35) (layer "B.Cu") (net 1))
 (segment (start 57.456 82.84) (end 60.833 82.84) (width 0.35) (layer "B.Cu") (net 1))
 (segment (start 60.833 82.84) (end 63.956 82.84) (width 0.35) (layer "B.Cu") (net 1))
 (segment (start 63.295 69.977) (end 58.166 69.977) (width 0.35) (layer "B.Cu") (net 1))
 (segment (start 75.998 82.713) (end 69.378 82.713) (width 0.35) (layer "B.Cu") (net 6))
 (segment (start 58.674 79.883) (end 58.674 72.009) (width 0.35) (layer "B.Cu") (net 6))
 (segment (start 82.498 82.713) (end 75.998 82.713) (width 0.35) (layer "B.Cu") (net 6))
 (segment (start 66.929 80.264) (end 59.055 80.264) (width 0.35) (layer "B.Cu") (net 6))
 (segment (start 69.378 82.713) (end 66.929 80.264) (width 0.35) (layer "B.Cu") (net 6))
 (segment (start 59.436 71.247) (end 63.295 71.247) (width 0.35) (layer "B.Cu") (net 6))
 (segment (start 59.055 80.264) (end 58.674 79.883) (width 0.35) (layer "B.Cu") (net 6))
 (segment (start 58.674 72.009) (end 59.436 71.247) (width 0.35) (layer "B.Cu") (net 6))
 (segment (start 84.582 75.311) (end 84.582 76.581) (width 0.35) (layer "B.Cu") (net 12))
 (segment (start 80.518 71.247) (end 84.582 75.311) (width 0.35) (layer "B.Cu") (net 12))
 (segment (start 84.582 76.581) (end 85.09 77.089) (width 0.35) (layer "B.Cu") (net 12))
 (segment (start 72.595 71.247) (end 80.518 71.247) (width 0.35) (layer "B.Cu") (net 12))
 (segment (start 85.09 77.089) (end 87.381 77.089) (width 0.35) (layer "B.Cu") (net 12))
 (segment (start 79.629 72.517) (end 82.042 74.93) (width 0.35) (layer "B.Cu") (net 13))
 (segment (start 83.312 79.629) (end 83.312 79.883) (width 0.35) (layer "B.Cu") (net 13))
 (segment (start 83.312 79.883) (end 83.947 80.518) (width 0.35) (layer "B.Cu") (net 13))
 (segment (start 83.312 76.2) (end 83.312 79.629) (width 0.35) (layer "B.Cu") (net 13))
 (segment (start 82.042 74.93) (end 83.312 76.2) (width 0.35) (layer "B.Cu") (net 13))
 (segment (start 87.381 80.772) (end 84.201 80.772) (width 0.35) (layer "B.Cu") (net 13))
 (segment (start 84.201 80.772) (end 83.947 80.518) (width 0.35) (layer "B.Cu") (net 13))
 (segment (start 72.595 72.517) (end 79.629 72.517) (width 0.35) (layer "B.Cu") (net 13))
 (segment (start 72.595 64.897) (end 74.422 64.897) (width 0.35) (layer "B.Cu") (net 7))
 (segment (start 75.946 63.373) (end 76.611 63.373) (width 0.35) (layer "B.Cu") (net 7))
 (segment (start 74.422 64.897) (end 75.946 63.373) (width 0.35) (layer "B.Cu") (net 7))
 (segment (start 72.595 66.167) (end 78.232 66.167) (width 0.35) (layer "B.Cu") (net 8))
 (segment (start 78.867 63.373) (end 78.613 63.627) (width 0.35) (layer "B.Cu") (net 8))
 (segment (start 80.137 63.373) (end 78.867 63.373) (width 0.35) (layer "B.Cu") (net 8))
 (segment (start 78.613 63.627) (end 78.613 65.786) (width 0.35) (layer "B.Cu") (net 8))
 (segment (start 78.613 65.786) (end 78.232 66.167) (width 0.35) (layer "B.Cu") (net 8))
 (segment (start 81.915 66.802) (end 81.28 67.437) (width 0.35) (layer "B.Cu") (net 9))
 (segment (start 81.28 67.437) (end 72.595 67.437) (width 0.35) (layer "B.Cu") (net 9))
 (segment (start 83.439 63.373) (end 82.169 63.373) (width 0.35) (layer "B.Cu") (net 9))
 (segment (start 81.915 63.627) (end 81.915 66.802) (width 0.35) (layer "B.Cu") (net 9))
 (segment (start 82.169 63.373) (end 81.915 63.627) (width 0.35) (layer "B.Cu") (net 9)))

